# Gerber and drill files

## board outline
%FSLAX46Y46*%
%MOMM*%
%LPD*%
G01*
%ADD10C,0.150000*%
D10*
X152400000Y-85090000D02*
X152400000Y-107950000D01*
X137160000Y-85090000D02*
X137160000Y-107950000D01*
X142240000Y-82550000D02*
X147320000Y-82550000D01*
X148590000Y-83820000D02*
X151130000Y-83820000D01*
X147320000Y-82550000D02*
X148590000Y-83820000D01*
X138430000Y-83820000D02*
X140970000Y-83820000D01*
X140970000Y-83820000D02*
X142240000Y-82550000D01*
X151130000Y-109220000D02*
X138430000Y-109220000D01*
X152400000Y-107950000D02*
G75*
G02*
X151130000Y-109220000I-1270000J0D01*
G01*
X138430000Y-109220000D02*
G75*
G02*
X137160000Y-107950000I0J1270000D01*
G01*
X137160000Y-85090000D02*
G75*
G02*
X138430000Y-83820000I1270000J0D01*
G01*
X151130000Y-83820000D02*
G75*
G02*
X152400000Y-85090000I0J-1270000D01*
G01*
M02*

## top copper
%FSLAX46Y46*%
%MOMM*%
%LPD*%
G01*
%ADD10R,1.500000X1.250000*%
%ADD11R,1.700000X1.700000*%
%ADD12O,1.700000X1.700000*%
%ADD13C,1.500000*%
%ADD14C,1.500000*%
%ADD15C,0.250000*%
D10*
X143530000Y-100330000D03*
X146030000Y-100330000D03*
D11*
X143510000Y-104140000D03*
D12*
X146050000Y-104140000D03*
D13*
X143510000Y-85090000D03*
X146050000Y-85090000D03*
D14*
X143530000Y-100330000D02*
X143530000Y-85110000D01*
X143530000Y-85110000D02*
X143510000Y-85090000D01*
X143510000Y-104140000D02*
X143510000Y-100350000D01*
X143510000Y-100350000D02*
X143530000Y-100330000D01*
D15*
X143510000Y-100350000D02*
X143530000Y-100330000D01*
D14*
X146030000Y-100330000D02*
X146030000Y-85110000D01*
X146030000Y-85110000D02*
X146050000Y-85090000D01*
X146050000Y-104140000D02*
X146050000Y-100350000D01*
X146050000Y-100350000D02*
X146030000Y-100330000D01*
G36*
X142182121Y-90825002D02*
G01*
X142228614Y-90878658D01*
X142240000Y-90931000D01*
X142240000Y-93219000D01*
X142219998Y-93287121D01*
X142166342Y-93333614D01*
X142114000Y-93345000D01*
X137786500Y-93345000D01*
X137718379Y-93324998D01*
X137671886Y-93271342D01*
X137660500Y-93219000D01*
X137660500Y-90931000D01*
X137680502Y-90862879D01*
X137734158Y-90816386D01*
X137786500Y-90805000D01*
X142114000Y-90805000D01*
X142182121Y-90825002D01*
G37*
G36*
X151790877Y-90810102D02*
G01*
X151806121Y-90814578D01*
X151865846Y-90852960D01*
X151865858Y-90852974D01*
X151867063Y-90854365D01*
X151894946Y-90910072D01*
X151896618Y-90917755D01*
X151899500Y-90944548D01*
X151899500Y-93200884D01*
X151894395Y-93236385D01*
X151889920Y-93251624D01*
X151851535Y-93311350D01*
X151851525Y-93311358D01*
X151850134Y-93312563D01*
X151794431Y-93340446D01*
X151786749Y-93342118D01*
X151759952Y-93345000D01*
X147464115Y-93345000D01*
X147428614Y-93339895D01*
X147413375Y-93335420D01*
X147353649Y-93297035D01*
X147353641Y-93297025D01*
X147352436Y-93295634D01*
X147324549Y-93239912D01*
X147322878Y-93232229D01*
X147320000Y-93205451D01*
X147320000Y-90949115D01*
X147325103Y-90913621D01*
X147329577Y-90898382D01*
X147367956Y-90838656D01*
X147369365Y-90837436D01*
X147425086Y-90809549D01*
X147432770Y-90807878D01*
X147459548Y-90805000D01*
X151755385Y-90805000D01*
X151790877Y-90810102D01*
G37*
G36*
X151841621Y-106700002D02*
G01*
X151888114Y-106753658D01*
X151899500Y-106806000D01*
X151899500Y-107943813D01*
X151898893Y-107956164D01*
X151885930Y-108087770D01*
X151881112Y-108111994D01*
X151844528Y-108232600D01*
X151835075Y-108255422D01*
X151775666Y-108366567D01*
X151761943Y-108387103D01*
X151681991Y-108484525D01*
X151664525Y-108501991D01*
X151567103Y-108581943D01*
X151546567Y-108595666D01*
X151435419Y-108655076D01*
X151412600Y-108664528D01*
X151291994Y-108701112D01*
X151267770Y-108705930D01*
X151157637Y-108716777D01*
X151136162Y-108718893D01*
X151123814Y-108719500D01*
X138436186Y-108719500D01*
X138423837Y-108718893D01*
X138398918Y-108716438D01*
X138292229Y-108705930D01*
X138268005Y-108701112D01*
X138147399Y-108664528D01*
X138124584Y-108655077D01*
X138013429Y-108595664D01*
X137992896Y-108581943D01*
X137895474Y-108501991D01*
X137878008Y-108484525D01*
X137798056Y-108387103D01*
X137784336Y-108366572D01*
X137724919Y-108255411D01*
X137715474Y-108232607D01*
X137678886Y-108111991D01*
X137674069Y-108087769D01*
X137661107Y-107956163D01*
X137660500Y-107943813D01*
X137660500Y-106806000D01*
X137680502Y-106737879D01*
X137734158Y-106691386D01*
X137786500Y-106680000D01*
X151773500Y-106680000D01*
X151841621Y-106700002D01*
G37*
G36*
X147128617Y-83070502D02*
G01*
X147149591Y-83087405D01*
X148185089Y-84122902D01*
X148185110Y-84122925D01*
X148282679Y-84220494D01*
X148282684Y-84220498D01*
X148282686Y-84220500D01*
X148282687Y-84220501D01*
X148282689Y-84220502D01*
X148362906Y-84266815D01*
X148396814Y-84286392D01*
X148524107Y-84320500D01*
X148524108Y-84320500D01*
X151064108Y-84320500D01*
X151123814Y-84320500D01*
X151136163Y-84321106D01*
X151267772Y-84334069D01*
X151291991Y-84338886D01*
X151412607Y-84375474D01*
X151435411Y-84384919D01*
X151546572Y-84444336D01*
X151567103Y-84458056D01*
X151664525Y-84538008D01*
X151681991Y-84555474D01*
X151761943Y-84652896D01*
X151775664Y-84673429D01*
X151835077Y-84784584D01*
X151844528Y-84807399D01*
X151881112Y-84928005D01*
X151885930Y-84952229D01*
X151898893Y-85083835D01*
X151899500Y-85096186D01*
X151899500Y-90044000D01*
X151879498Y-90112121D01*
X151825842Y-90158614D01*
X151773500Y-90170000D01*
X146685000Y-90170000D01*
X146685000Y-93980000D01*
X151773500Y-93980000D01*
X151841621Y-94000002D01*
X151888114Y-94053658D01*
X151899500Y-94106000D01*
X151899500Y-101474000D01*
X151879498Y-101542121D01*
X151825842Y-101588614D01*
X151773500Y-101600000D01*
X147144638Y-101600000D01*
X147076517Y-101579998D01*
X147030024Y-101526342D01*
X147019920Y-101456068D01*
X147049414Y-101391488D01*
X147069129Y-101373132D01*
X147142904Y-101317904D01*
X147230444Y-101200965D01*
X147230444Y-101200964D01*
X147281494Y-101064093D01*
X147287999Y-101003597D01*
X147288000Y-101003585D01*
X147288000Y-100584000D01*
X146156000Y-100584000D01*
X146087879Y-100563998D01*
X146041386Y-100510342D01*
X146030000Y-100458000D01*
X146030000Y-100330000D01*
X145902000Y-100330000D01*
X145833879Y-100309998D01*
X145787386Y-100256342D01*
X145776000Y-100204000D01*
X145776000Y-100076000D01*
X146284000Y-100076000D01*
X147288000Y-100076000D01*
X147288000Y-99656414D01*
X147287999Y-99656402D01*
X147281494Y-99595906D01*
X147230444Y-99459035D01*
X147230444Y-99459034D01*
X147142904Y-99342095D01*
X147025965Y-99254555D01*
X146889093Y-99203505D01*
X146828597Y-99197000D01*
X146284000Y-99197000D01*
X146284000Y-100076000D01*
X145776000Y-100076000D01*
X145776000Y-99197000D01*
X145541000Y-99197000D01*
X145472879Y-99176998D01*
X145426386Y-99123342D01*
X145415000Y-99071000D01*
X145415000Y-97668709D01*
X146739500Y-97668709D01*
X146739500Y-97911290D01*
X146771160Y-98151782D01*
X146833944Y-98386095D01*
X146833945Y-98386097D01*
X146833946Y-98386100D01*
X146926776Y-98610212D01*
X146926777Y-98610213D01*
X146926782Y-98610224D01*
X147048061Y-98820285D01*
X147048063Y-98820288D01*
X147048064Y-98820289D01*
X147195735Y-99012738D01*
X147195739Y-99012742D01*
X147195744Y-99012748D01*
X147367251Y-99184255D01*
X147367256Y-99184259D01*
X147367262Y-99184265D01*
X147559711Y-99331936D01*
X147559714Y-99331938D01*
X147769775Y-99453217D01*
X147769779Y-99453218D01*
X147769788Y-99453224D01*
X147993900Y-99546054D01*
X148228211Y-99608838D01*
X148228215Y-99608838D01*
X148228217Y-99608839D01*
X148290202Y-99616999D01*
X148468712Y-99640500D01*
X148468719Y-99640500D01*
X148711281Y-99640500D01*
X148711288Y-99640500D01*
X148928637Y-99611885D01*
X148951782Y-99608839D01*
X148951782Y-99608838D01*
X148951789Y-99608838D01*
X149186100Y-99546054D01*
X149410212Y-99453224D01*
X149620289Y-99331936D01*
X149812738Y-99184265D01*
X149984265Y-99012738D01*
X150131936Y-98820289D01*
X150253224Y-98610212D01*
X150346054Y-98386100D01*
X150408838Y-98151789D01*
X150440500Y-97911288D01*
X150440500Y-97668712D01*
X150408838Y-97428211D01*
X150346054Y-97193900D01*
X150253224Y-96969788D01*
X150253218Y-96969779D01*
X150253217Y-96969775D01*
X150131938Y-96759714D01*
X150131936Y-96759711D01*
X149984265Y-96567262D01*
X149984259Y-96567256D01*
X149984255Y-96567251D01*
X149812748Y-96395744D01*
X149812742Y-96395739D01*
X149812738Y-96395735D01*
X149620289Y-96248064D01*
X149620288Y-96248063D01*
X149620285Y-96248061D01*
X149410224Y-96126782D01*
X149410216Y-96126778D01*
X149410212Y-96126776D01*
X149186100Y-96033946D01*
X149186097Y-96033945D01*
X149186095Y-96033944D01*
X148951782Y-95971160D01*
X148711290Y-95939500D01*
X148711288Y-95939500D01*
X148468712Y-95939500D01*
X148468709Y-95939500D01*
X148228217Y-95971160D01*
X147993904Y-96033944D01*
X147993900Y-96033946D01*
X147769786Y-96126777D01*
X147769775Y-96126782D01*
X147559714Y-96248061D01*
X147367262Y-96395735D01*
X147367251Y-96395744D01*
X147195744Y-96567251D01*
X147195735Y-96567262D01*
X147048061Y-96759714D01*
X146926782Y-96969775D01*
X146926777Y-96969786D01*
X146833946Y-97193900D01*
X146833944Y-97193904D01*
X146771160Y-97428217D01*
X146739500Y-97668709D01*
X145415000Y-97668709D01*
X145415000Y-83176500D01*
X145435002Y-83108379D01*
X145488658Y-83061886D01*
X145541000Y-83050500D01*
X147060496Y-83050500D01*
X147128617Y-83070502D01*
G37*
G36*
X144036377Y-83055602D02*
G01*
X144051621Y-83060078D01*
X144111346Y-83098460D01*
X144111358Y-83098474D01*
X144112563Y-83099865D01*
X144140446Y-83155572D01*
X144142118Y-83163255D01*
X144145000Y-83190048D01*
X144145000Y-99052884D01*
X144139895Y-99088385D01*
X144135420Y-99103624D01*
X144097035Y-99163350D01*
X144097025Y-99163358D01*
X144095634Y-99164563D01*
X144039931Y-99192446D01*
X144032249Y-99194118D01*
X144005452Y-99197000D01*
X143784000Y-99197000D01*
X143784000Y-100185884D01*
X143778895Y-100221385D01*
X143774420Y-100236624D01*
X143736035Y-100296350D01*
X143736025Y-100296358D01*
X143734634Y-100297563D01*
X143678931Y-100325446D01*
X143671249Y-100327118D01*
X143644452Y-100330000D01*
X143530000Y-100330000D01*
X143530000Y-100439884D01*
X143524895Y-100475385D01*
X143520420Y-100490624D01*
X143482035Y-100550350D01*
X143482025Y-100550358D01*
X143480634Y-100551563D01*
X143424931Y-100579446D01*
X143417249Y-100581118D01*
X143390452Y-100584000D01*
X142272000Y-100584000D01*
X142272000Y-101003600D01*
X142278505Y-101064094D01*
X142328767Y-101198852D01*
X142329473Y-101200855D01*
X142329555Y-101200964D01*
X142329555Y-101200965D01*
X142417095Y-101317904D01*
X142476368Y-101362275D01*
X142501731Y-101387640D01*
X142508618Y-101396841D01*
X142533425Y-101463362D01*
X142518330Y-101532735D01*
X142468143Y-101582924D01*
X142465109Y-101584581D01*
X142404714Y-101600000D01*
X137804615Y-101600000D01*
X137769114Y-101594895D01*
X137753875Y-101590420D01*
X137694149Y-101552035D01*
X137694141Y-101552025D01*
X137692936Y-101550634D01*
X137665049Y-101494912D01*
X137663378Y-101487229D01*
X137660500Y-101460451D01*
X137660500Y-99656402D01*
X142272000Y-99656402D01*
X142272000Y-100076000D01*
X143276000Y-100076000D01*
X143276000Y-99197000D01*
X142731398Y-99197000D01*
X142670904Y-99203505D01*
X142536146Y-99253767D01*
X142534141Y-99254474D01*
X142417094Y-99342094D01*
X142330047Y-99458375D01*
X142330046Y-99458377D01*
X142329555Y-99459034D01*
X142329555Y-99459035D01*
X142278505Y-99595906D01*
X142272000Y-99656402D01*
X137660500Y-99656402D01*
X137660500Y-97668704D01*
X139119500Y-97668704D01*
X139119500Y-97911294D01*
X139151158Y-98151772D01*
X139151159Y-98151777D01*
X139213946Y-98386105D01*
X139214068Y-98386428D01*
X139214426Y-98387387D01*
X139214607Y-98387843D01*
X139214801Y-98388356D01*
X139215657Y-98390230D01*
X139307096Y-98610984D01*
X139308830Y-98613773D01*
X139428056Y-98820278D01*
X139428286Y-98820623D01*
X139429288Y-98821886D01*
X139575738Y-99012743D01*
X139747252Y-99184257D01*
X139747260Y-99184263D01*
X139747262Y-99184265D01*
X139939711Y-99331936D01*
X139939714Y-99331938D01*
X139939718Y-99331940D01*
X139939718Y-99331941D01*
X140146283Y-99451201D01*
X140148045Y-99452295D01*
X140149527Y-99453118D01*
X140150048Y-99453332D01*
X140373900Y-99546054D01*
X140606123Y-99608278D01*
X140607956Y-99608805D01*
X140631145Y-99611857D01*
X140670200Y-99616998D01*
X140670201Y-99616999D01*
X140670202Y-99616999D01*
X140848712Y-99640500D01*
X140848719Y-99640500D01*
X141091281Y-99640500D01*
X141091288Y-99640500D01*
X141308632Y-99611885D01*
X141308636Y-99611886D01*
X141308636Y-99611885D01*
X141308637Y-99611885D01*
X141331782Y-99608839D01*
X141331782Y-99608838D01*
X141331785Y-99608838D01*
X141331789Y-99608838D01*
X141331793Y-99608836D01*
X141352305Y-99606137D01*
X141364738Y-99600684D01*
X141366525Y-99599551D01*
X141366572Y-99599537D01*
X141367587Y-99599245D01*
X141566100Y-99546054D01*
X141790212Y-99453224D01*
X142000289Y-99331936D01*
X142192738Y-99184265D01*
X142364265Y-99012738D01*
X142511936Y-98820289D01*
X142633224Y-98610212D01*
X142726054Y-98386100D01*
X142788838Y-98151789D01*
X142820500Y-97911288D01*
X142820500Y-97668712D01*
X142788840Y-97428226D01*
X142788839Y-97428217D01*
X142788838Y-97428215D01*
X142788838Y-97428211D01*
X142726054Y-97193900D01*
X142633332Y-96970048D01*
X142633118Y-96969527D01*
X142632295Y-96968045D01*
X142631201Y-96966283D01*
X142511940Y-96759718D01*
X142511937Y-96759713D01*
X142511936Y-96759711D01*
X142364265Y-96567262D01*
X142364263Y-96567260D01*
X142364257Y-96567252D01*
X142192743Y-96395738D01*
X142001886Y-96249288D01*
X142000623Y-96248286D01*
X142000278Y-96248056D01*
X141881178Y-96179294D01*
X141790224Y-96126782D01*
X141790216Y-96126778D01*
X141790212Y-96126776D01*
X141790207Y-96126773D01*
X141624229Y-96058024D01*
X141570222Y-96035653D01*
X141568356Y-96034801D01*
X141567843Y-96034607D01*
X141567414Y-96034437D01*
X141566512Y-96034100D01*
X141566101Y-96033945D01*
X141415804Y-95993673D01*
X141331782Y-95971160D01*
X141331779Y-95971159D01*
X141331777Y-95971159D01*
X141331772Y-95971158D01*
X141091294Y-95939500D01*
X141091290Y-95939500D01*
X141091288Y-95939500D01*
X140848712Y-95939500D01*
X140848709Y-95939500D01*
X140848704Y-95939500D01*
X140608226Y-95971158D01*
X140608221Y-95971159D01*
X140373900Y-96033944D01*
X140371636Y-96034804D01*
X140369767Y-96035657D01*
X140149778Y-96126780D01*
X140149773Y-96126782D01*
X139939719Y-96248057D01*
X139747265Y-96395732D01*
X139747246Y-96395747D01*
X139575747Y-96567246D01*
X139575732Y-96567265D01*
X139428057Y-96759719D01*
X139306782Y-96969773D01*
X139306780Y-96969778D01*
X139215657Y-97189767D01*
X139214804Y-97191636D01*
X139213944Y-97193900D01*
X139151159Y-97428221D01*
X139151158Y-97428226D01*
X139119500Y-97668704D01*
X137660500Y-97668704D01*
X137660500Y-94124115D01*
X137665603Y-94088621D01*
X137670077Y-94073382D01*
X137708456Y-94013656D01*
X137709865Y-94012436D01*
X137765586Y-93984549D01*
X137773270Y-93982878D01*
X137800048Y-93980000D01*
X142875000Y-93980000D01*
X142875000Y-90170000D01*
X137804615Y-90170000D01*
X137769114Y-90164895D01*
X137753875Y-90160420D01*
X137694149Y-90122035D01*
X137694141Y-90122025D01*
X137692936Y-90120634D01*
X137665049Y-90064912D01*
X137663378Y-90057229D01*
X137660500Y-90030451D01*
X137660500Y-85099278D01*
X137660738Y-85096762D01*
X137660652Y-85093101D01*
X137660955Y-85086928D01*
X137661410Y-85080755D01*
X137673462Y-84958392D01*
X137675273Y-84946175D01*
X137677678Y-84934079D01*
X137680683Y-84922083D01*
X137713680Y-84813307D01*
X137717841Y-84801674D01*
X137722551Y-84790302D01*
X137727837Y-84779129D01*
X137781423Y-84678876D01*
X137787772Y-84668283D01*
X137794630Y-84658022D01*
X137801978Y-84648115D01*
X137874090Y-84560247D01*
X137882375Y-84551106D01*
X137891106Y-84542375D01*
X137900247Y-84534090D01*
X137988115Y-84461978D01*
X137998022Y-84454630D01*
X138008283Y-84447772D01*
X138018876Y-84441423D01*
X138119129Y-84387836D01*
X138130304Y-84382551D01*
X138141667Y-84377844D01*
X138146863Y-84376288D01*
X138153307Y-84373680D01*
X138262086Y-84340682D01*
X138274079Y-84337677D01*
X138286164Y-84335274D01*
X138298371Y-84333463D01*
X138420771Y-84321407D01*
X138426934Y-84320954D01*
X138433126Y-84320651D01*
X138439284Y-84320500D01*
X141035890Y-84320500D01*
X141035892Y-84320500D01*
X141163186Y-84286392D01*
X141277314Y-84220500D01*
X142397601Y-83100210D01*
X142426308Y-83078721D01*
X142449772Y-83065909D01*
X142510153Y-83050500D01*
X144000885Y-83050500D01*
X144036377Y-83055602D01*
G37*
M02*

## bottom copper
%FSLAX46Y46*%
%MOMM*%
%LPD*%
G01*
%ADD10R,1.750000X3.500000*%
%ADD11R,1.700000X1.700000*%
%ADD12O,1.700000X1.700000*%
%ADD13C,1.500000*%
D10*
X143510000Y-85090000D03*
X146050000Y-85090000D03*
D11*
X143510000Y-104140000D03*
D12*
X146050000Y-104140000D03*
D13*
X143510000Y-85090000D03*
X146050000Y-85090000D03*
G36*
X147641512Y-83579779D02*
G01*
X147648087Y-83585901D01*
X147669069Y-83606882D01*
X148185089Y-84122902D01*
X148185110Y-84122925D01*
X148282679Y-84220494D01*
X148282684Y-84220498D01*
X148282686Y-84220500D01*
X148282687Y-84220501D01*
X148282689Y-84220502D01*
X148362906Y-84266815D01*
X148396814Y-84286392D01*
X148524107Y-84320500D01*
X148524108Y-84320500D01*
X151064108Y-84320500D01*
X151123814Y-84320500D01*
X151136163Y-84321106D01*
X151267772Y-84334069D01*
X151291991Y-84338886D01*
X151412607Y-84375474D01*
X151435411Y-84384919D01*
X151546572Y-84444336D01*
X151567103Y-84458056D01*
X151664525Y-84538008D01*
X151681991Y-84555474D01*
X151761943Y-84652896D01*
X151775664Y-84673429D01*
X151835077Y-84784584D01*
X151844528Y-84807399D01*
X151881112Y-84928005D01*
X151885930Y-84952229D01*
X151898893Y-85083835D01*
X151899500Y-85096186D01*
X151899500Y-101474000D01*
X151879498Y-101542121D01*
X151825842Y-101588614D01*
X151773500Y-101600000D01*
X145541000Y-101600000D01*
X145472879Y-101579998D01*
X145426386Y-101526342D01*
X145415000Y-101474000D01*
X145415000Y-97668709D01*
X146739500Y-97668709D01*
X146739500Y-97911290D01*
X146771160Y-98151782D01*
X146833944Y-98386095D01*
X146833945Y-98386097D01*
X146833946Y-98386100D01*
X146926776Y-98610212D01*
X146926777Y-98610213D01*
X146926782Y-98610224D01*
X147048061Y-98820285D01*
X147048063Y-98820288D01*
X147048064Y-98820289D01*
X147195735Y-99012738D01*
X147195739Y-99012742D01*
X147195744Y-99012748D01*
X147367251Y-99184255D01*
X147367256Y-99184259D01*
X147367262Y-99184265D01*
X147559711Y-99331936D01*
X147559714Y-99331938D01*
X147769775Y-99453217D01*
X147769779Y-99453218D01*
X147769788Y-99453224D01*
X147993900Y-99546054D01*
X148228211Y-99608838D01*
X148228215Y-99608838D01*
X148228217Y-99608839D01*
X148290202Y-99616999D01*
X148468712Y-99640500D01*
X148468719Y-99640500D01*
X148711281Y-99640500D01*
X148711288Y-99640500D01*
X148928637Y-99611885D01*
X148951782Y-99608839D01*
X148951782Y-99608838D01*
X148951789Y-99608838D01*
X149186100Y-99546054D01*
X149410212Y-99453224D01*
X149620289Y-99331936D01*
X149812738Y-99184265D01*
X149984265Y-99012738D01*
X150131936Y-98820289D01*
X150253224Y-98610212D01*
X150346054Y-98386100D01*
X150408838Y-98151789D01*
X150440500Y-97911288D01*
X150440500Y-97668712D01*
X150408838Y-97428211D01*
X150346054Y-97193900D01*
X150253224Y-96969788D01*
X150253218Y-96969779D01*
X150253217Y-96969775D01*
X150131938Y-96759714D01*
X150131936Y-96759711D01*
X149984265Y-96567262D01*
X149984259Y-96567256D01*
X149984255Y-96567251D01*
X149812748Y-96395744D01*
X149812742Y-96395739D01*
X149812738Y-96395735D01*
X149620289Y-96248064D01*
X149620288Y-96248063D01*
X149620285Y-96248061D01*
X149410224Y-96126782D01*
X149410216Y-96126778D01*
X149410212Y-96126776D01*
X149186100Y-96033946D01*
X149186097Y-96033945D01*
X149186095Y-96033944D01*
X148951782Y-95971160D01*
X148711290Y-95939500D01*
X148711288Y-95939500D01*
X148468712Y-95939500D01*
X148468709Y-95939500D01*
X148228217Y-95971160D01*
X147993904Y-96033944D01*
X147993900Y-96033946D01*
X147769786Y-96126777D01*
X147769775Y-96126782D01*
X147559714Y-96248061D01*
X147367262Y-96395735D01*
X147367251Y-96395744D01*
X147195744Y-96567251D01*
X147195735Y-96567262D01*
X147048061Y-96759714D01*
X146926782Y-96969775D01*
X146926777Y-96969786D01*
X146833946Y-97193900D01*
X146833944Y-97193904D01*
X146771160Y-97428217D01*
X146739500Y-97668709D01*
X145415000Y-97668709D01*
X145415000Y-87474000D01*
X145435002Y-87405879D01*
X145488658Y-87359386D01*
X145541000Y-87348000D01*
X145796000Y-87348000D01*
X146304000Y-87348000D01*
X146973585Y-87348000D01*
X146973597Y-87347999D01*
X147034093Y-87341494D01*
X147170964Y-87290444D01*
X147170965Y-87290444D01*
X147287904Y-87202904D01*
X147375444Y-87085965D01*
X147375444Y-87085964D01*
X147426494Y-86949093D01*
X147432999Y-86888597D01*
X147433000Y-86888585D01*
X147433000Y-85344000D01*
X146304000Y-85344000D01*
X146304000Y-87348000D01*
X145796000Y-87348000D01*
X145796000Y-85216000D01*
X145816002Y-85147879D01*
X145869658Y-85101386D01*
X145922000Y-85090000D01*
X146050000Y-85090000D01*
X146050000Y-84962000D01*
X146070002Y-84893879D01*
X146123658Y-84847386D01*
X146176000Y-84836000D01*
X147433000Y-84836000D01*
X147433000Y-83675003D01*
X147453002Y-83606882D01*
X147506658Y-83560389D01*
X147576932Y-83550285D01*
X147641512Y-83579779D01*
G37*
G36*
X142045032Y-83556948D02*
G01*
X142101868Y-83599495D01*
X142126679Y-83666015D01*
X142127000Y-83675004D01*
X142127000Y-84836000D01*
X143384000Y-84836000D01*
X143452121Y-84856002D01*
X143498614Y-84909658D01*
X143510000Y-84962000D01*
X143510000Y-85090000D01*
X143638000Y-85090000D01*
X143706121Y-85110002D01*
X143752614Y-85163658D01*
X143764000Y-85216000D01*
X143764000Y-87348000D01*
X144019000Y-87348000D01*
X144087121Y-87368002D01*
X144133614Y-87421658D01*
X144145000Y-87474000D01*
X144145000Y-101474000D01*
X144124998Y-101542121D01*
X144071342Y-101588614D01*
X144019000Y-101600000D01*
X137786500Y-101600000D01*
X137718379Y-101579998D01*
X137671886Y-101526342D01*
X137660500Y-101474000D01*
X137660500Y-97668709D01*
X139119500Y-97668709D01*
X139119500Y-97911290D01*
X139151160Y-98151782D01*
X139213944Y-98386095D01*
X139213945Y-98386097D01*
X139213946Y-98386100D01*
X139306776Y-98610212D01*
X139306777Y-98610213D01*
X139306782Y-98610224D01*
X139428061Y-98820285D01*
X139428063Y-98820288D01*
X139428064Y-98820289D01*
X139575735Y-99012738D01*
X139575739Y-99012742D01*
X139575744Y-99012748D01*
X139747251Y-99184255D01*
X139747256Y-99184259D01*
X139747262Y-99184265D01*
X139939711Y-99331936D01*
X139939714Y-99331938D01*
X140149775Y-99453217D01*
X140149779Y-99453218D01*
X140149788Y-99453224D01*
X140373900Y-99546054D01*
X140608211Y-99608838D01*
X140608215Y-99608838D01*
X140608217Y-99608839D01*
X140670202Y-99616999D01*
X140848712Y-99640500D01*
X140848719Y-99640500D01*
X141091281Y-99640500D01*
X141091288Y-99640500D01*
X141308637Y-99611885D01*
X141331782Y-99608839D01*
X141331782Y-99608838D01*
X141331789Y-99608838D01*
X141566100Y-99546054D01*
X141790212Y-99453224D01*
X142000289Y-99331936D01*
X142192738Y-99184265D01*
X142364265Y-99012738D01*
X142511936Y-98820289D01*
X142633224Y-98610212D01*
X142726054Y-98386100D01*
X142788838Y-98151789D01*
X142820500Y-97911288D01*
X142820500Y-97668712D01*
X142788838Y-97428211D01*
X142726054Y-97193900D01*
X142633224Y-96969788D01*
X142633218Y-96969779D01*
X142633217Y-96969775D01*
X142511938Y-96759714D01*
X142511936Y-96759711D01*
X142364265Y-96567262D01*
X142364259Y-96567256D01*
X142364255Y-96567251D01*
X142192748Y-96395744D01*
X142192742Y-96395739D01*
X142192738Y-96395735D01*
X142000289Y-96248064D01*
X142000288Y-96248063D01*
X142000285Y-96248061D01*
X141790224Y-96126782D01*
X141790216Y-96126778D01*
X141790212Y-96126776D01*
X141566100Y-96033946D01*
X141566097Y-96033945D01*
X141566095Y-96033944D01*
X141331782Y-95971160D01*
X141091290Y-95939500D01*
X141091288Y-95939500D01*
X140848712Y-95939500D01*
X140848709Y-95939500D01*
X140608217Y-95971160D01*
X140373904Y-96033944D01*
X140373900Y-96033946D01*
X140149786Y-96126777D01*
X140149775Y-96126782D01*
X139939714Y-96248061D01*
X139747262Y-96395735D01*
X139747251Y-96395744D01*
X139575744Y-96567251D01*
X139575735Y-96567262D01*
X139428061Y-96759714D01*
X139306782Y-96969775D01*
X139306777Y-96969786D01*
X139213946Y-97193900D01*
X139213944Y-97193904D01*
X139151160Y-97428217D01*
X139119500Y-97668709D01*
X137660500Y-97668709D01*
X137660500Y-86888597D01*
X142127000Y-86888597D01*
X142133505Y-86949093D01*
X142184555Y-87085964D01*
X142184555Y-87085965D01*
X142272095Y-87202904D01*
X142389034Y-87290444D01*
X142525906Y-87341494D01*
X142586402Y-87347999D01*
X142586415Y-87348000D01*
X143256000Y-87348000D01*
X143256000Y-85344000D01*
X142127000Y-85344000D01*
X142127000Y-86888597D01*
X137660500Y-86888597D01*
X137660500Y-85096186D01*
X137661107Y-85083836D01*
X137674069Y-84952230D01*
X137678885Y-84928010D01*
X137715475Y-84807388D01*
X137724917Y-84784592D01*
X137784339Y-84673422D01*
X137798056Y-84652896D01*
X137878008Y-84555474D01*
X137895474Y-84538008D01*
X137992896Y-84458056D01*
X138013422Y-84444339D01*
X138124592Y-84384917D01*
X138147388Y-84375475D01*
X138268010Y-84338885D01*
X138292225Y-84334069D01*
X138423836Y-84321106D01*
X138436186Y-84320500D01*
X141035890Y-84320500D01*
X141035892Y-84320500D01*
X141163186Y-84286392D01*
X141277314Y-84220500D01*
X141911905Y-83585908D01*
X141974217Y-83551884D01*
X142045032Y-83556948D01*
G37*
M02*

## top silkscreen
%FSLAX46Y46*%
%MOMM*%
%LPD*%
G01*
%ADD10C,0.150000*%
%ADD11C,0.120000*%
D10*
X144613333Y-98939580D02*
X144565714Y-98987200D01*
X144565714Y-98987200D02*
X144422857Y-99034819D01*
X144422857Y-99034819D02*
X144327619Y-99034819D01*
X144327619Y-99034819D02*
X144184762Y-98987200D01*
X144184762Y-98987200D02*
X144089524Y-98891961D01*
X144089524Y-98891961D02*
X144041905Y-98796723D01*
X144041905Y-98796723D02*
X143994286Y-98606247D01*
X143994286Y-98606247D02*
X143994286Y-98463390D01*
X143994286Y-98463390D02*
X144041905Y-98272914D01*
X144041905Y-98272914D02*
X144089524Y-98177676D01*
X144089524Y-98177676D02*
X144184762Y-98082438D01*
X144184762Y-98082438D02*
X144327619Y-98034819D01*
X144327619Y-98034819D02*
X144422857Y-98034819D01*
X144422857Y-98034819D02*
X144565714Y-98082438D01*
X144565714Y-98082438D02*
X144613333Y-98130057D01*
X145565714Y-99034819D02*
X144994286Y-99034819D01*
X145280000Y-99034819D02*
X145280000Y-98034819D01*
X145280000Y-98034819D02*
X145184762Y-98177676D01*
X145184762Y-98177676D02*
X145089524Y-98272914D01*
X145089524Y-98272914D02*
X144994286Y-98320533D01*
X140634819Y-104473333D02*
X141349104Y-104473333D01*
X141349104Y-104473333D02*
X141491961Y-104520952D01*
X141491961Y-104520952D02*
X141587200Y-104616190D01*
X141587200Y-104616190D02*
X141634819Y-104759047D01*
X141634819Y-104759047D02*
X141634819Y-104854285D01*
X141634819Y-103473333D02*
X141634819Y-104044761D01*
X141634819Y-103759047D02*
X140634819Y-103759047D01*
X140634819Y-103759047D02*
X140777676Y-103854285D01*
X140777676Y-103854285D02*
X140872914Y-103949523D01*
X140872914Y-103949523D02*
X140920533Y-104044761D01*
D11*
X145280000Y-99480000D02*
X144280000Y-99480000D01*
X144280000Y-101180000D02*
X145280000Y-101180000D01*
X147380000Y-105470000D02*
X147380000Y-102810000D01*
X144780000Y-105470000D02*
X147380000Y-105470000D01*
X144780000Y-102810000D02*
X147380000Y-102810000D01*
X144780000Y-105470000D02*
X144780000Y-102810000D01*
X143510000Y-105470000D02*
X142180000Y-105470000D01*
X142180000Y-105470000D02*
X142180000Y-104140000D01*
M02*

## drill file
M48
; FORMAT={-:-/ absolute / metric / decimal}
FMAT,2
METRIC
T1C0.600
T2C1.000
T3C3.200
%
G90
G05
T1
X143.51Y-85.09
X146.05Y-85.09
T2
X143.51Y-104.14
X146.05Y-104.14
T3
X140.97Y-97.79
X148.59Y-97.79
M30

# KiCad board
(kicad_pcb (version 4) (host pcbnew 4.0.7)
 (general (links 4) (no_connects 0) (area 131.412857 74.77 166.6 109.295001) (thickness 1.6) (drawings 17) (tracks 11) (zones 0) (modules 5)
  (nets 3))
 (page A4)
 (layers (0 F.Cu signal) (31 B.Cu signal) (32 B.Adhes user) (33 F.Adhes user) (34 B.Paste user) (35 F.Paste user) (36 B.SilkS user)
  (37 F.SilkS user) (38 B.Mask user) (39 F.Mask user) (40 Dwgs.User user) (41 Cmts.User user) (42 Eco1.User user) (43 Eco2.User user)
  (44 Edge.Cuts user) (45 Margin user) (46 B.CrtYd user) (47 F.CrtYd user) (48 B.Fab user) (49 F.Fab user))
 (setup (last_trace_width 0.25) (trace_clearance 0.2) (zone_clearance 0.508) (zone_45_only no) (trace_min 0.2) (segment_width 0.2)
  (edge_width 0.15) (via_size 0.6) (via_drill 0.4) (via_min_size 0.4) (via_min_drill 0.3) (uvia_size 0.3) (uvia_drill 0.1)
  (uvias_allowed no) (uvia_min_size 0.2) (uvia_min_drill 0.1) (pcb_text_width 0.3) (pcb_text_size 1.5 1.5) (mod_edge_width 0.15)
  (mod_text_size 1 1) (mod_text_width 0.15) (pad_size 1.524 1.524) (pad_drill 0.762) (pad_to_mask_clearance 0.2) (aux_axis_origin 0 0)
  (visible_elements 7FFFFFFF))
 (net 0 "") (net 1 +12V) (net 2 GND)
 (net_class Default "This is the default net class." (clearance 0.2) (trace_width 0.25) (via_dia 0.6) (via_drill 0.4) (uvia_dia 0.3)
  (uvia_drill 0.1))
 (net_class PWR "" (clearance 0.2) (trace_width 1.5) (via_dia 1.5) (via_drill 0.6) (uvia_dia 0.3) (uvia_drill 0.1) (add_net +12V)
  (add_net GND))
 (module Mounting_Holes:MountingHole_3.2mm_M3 (layer F.Cu) (at 140.97 97.79)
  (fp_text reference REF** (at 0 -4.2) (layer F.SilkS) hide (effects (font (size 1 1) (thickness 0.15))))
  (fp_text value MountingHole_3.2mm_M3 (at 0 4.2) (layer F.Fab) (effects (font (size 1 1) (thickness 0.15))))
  (pad 1 np_thru_hole circle (at 0 0) (size 3.2 3.2) (drill 3.2) (layers *.Cu *.Mask)))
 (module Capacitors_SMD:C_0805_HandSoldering (layer F.Cu) (at 144.78 100.33)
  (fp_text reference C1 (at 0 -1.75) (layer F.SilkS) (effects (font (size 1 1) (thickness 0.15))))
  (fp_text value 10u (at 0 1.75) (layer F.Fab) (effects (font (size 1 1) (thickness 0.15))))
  (fp_line (start 0.5 -0.85) (end -0.5 -0.85) (layer F.SilkS) (width 0.12))
  (fp_line (start -0.5 0.85) (end 0.5 0.85) (layer F.SilkS) (width 0.12))
  (pad 1 smd rect (at -1.25 0) (size 1.5 1.25) (layers F.Cu F.Paste F.Mask) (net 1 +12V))
  (pad 2 smd rect (at 1.25 0) (size 1.5 1.25) (layers F.Cu F.Paste F.Mask) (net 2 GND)))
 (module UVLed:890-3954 (layer B.Cu) (at 144.78 85.09)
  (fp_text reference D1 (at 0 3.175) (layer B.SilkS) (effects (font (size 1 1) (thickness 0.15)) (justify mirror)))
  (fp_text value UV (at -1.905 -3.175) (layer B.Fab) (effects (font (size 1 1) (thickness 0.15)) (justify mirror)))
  (pad 2 smd rect (at -1.27 0) (size 1.75 3.5) (layers B.Cu B.Paste B.Mask) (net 1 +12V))
  (pad 1 smd rect (at 1.27 0) (size 1.75 3.5) (layers B.Cu B.Paste B.Mask) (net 2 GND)))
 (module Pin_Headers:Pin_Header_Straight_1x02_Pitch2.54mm (layer F.Cu) (at 143.51 104.14 90)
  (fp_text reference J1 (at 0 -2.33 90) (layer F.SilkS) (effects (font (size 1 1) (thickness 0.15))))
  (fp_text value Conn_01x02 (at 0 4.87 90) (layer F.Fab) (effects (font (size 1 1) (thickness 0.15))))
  (fp_line (start -1.33 3.87) (end 1.33 3.87) (layer F.SilkS) (width 0.12))
  (fp_line (start -1.33 1.27) (end -1.33 3.87) (layer F.SilkS) (width 0.12))
  (fp_line (start 1.33 1.27) (end 1.33 3.87) (layer F.SilkS) (width 0.12))
  (fp_line (start -1.33 1.27) (end 1.33 1.27) (layer F.SilkS) (width 0.12))
  (fp_line (start -1.33 0) (end -1.33 -1.33) (layer F.SilkS) (width 0.12))
  (fp_line (start -1.33 -1.33) (end 0 -1.33) (layer F.SilkS) (width 0.12))
  (pad 1 thru_hole rect (at 0 0 90) (size 1.7 1.7) (drill 1) (layers *.Cu *.Mask) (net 1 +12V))
  (pad 2 thru_hole oval (at 0 2.54 90) (size 1.7 1.7) (drill 1) (layers *.Cu *.Mask) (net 2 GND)))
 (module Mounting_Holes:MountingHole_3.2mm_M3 (layer F.Cu) (at 148.59 97.79)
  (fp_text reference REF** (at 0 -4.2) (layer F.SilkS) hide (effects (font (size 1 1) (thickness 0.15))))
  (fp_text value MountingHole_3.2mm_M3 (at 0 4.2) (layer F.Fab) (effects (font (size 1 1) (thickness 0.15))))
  (pad 1 np_thru_hole circle (at 0 0) (size 3.2 3.2) (drill 3.2) (layers *.Cu *.Mask)))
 (gr_line (start 152.4 85.09) (end 152.4 107.95) (angle 90) (layer Edge.Cuts) (width 0.15))
 (gr_line (start 137.16 85.09) (end 137.16 107.95) (angle 90) (layer Edge.Cuts) (width 0.15))
 (gr_line (start 142.24 82.55) (end 147.32 82.55) (angle 90) (layer Edge.Cuts) (width 0.15))
 (gr_line (start 148.59 83.82) (end 151.13 83.82) (angle 90) (layer Edge.Cuts) (width 0.15))
 (gr_line (start 147.32 82.55) (end 148.59 83.82) (angle 90) (layer Edge.Cuts) (width 0.15))
 (gr_line (start 138.43 83.82) (end 140.97 83.82) (angle 90) (layer Edge.Cuts) (width 0.15))
 (gr_line (start 140.97 83.82) (end 142.24 82.55) (angle 90) (layer Edge.Cuts) (width 0.15))
 (gr_line (start 151.13 109.22) (end 138.43 109.22) (angle 90) (layer Edge.Cuts) (width 0.15))
 (gr_arc (start 151.13 107.95) (end 152.4 107.95) (angle 90) (layer Edge.Cuts) (width 0.15))
 (gr_arc (start 138.43 107.95) (end 138.43 109.22) (angle 90) (layer Edge.Cuts) (width 0.15))
 (gr_arc (start 138.43 85.09) (end 137.16 85.09) (angle 90) (layer Edge.Cuts) (width 0.15))
 (gr_arc (start 151.13 85.09) (end 151.13 83.82) (angle 90) (layer Edge.Cuts) (width 0.15))
 (segment (start 143.53 100.33) (end 143.53 85.11) (width 1.5) (layer F.Cu) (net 1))
 (via (at 143.51 85.09) (size 1.5) (drill 0.6) (layers F.Cu B.Cu) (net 1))
 (segment (start 143.53 85.11) (end 143.51 85.09) (width 1.5) (layer F.Cu) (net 1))
 (segment (start 143.51 104.14) (end 143.51 100.35) (width 1.5) (layer F.Cu) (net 1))
 (segment (start 143.51 100.35) (end 143.53 100.33) (width 1.5) (layer F.Cu) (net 1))
 (segment (start 143.51 100.35) (end 143.53 100.33) (width 0.25) (layer F.Cu) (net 1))
 (segment (start 146.03 100.33) (end 146.03 85.11) (width 1.5) (layer F.Cu) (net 2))
 (via (at 146.05 85.09) (size 1.5) (drill 0.6) (layers F.Cu B.Cu) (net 2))
 (segment (start 146.03 85.11) (end 146.05 85.09) (width 1.5) (layer F.Cu) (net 2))
 (segment (start 146.05 104.14) (end 146.05 100.35) (width 1.5) (layer F.Cu) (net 2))
 (segment (start 146.05 100.35) (end 146.03 100.33) (width 1.5) (layer F.Cu) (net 2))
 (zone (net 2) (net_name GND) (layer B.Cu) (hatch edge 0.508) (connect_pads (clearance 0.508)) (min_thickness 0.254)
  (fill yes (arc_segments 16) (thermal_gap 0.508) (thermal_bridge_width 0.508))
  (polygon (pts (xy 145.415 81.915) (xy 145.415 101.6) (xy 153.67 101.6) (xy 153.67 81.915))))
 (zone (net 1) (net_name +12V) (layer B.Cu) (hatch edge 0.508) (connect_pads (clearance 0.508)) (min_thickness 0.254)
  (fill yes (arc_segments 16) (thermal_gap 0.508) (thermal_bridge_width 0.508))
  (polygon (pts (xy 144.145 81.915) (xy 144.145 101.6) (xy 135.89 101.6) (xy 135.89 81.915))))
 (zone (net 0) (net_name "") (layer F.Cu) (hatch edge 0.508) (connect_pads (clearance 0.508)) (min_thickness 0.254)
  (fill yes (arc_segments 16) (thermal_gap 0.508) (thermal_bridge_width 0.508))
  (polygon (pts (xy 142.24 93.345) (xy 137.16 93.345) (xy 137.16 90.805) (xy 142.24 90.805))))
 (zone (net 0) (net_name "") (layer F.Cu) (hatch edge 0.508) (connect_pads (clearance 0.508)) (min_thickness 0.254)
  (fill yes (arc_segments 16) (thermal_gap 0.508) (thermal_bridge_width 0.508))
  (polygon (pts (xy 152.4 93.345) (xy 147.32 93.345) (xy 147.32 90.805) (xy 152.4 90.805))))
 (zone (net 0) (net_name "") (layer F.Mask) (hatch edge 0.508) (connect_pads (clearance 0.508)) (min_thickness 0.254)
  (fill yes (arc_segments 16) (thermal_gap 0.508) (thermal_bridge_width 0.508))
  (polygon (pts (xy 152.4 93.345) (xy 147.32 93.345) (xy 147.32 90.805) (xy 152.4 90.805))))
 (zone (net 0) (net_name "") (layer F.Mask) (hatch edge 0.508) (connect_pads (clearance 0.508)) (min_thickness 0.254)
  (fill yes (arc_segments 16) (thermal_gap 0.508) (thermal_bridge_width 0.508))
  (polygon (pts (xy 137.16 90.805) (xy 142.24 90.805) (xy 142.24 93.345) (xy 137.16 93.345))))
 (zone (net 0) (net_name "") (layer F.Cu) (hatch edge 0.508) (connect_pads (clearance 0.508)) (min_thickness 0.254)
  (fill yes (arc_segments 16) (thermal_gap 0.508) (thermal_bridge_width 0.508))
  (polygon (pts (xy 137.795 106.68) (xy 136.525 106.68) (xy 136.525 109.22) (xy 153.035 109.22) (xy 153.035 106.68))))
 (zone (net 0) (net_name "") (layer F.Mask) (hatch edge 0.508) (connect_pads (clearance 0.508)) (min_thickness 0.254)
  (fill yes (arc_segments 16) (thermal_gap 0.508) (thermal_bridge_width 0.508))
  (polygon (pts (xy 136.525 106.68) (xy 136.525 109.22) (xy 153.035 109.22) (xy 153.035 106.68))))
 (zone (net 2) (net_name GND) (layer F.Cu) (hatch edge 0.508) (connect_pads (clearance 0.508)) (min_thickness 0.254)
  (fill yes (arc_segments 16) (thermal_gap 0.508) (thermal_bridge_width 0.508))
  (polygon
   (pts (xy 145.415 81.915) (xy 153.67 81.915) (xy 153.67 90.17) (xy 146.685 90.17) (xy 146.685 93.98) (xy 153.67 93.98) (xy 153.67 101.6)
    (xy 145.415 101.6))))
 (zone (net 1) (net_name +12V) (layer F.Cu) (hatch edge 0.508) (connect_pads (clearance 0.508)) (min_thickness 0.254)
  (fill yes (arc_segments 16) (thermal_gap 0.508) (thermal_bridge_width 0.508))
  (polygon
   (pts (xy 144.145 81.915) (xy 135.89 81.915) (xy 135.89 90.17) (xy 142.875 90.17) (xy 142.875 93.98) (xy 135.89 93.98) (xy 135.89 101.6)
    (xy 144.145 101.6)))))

